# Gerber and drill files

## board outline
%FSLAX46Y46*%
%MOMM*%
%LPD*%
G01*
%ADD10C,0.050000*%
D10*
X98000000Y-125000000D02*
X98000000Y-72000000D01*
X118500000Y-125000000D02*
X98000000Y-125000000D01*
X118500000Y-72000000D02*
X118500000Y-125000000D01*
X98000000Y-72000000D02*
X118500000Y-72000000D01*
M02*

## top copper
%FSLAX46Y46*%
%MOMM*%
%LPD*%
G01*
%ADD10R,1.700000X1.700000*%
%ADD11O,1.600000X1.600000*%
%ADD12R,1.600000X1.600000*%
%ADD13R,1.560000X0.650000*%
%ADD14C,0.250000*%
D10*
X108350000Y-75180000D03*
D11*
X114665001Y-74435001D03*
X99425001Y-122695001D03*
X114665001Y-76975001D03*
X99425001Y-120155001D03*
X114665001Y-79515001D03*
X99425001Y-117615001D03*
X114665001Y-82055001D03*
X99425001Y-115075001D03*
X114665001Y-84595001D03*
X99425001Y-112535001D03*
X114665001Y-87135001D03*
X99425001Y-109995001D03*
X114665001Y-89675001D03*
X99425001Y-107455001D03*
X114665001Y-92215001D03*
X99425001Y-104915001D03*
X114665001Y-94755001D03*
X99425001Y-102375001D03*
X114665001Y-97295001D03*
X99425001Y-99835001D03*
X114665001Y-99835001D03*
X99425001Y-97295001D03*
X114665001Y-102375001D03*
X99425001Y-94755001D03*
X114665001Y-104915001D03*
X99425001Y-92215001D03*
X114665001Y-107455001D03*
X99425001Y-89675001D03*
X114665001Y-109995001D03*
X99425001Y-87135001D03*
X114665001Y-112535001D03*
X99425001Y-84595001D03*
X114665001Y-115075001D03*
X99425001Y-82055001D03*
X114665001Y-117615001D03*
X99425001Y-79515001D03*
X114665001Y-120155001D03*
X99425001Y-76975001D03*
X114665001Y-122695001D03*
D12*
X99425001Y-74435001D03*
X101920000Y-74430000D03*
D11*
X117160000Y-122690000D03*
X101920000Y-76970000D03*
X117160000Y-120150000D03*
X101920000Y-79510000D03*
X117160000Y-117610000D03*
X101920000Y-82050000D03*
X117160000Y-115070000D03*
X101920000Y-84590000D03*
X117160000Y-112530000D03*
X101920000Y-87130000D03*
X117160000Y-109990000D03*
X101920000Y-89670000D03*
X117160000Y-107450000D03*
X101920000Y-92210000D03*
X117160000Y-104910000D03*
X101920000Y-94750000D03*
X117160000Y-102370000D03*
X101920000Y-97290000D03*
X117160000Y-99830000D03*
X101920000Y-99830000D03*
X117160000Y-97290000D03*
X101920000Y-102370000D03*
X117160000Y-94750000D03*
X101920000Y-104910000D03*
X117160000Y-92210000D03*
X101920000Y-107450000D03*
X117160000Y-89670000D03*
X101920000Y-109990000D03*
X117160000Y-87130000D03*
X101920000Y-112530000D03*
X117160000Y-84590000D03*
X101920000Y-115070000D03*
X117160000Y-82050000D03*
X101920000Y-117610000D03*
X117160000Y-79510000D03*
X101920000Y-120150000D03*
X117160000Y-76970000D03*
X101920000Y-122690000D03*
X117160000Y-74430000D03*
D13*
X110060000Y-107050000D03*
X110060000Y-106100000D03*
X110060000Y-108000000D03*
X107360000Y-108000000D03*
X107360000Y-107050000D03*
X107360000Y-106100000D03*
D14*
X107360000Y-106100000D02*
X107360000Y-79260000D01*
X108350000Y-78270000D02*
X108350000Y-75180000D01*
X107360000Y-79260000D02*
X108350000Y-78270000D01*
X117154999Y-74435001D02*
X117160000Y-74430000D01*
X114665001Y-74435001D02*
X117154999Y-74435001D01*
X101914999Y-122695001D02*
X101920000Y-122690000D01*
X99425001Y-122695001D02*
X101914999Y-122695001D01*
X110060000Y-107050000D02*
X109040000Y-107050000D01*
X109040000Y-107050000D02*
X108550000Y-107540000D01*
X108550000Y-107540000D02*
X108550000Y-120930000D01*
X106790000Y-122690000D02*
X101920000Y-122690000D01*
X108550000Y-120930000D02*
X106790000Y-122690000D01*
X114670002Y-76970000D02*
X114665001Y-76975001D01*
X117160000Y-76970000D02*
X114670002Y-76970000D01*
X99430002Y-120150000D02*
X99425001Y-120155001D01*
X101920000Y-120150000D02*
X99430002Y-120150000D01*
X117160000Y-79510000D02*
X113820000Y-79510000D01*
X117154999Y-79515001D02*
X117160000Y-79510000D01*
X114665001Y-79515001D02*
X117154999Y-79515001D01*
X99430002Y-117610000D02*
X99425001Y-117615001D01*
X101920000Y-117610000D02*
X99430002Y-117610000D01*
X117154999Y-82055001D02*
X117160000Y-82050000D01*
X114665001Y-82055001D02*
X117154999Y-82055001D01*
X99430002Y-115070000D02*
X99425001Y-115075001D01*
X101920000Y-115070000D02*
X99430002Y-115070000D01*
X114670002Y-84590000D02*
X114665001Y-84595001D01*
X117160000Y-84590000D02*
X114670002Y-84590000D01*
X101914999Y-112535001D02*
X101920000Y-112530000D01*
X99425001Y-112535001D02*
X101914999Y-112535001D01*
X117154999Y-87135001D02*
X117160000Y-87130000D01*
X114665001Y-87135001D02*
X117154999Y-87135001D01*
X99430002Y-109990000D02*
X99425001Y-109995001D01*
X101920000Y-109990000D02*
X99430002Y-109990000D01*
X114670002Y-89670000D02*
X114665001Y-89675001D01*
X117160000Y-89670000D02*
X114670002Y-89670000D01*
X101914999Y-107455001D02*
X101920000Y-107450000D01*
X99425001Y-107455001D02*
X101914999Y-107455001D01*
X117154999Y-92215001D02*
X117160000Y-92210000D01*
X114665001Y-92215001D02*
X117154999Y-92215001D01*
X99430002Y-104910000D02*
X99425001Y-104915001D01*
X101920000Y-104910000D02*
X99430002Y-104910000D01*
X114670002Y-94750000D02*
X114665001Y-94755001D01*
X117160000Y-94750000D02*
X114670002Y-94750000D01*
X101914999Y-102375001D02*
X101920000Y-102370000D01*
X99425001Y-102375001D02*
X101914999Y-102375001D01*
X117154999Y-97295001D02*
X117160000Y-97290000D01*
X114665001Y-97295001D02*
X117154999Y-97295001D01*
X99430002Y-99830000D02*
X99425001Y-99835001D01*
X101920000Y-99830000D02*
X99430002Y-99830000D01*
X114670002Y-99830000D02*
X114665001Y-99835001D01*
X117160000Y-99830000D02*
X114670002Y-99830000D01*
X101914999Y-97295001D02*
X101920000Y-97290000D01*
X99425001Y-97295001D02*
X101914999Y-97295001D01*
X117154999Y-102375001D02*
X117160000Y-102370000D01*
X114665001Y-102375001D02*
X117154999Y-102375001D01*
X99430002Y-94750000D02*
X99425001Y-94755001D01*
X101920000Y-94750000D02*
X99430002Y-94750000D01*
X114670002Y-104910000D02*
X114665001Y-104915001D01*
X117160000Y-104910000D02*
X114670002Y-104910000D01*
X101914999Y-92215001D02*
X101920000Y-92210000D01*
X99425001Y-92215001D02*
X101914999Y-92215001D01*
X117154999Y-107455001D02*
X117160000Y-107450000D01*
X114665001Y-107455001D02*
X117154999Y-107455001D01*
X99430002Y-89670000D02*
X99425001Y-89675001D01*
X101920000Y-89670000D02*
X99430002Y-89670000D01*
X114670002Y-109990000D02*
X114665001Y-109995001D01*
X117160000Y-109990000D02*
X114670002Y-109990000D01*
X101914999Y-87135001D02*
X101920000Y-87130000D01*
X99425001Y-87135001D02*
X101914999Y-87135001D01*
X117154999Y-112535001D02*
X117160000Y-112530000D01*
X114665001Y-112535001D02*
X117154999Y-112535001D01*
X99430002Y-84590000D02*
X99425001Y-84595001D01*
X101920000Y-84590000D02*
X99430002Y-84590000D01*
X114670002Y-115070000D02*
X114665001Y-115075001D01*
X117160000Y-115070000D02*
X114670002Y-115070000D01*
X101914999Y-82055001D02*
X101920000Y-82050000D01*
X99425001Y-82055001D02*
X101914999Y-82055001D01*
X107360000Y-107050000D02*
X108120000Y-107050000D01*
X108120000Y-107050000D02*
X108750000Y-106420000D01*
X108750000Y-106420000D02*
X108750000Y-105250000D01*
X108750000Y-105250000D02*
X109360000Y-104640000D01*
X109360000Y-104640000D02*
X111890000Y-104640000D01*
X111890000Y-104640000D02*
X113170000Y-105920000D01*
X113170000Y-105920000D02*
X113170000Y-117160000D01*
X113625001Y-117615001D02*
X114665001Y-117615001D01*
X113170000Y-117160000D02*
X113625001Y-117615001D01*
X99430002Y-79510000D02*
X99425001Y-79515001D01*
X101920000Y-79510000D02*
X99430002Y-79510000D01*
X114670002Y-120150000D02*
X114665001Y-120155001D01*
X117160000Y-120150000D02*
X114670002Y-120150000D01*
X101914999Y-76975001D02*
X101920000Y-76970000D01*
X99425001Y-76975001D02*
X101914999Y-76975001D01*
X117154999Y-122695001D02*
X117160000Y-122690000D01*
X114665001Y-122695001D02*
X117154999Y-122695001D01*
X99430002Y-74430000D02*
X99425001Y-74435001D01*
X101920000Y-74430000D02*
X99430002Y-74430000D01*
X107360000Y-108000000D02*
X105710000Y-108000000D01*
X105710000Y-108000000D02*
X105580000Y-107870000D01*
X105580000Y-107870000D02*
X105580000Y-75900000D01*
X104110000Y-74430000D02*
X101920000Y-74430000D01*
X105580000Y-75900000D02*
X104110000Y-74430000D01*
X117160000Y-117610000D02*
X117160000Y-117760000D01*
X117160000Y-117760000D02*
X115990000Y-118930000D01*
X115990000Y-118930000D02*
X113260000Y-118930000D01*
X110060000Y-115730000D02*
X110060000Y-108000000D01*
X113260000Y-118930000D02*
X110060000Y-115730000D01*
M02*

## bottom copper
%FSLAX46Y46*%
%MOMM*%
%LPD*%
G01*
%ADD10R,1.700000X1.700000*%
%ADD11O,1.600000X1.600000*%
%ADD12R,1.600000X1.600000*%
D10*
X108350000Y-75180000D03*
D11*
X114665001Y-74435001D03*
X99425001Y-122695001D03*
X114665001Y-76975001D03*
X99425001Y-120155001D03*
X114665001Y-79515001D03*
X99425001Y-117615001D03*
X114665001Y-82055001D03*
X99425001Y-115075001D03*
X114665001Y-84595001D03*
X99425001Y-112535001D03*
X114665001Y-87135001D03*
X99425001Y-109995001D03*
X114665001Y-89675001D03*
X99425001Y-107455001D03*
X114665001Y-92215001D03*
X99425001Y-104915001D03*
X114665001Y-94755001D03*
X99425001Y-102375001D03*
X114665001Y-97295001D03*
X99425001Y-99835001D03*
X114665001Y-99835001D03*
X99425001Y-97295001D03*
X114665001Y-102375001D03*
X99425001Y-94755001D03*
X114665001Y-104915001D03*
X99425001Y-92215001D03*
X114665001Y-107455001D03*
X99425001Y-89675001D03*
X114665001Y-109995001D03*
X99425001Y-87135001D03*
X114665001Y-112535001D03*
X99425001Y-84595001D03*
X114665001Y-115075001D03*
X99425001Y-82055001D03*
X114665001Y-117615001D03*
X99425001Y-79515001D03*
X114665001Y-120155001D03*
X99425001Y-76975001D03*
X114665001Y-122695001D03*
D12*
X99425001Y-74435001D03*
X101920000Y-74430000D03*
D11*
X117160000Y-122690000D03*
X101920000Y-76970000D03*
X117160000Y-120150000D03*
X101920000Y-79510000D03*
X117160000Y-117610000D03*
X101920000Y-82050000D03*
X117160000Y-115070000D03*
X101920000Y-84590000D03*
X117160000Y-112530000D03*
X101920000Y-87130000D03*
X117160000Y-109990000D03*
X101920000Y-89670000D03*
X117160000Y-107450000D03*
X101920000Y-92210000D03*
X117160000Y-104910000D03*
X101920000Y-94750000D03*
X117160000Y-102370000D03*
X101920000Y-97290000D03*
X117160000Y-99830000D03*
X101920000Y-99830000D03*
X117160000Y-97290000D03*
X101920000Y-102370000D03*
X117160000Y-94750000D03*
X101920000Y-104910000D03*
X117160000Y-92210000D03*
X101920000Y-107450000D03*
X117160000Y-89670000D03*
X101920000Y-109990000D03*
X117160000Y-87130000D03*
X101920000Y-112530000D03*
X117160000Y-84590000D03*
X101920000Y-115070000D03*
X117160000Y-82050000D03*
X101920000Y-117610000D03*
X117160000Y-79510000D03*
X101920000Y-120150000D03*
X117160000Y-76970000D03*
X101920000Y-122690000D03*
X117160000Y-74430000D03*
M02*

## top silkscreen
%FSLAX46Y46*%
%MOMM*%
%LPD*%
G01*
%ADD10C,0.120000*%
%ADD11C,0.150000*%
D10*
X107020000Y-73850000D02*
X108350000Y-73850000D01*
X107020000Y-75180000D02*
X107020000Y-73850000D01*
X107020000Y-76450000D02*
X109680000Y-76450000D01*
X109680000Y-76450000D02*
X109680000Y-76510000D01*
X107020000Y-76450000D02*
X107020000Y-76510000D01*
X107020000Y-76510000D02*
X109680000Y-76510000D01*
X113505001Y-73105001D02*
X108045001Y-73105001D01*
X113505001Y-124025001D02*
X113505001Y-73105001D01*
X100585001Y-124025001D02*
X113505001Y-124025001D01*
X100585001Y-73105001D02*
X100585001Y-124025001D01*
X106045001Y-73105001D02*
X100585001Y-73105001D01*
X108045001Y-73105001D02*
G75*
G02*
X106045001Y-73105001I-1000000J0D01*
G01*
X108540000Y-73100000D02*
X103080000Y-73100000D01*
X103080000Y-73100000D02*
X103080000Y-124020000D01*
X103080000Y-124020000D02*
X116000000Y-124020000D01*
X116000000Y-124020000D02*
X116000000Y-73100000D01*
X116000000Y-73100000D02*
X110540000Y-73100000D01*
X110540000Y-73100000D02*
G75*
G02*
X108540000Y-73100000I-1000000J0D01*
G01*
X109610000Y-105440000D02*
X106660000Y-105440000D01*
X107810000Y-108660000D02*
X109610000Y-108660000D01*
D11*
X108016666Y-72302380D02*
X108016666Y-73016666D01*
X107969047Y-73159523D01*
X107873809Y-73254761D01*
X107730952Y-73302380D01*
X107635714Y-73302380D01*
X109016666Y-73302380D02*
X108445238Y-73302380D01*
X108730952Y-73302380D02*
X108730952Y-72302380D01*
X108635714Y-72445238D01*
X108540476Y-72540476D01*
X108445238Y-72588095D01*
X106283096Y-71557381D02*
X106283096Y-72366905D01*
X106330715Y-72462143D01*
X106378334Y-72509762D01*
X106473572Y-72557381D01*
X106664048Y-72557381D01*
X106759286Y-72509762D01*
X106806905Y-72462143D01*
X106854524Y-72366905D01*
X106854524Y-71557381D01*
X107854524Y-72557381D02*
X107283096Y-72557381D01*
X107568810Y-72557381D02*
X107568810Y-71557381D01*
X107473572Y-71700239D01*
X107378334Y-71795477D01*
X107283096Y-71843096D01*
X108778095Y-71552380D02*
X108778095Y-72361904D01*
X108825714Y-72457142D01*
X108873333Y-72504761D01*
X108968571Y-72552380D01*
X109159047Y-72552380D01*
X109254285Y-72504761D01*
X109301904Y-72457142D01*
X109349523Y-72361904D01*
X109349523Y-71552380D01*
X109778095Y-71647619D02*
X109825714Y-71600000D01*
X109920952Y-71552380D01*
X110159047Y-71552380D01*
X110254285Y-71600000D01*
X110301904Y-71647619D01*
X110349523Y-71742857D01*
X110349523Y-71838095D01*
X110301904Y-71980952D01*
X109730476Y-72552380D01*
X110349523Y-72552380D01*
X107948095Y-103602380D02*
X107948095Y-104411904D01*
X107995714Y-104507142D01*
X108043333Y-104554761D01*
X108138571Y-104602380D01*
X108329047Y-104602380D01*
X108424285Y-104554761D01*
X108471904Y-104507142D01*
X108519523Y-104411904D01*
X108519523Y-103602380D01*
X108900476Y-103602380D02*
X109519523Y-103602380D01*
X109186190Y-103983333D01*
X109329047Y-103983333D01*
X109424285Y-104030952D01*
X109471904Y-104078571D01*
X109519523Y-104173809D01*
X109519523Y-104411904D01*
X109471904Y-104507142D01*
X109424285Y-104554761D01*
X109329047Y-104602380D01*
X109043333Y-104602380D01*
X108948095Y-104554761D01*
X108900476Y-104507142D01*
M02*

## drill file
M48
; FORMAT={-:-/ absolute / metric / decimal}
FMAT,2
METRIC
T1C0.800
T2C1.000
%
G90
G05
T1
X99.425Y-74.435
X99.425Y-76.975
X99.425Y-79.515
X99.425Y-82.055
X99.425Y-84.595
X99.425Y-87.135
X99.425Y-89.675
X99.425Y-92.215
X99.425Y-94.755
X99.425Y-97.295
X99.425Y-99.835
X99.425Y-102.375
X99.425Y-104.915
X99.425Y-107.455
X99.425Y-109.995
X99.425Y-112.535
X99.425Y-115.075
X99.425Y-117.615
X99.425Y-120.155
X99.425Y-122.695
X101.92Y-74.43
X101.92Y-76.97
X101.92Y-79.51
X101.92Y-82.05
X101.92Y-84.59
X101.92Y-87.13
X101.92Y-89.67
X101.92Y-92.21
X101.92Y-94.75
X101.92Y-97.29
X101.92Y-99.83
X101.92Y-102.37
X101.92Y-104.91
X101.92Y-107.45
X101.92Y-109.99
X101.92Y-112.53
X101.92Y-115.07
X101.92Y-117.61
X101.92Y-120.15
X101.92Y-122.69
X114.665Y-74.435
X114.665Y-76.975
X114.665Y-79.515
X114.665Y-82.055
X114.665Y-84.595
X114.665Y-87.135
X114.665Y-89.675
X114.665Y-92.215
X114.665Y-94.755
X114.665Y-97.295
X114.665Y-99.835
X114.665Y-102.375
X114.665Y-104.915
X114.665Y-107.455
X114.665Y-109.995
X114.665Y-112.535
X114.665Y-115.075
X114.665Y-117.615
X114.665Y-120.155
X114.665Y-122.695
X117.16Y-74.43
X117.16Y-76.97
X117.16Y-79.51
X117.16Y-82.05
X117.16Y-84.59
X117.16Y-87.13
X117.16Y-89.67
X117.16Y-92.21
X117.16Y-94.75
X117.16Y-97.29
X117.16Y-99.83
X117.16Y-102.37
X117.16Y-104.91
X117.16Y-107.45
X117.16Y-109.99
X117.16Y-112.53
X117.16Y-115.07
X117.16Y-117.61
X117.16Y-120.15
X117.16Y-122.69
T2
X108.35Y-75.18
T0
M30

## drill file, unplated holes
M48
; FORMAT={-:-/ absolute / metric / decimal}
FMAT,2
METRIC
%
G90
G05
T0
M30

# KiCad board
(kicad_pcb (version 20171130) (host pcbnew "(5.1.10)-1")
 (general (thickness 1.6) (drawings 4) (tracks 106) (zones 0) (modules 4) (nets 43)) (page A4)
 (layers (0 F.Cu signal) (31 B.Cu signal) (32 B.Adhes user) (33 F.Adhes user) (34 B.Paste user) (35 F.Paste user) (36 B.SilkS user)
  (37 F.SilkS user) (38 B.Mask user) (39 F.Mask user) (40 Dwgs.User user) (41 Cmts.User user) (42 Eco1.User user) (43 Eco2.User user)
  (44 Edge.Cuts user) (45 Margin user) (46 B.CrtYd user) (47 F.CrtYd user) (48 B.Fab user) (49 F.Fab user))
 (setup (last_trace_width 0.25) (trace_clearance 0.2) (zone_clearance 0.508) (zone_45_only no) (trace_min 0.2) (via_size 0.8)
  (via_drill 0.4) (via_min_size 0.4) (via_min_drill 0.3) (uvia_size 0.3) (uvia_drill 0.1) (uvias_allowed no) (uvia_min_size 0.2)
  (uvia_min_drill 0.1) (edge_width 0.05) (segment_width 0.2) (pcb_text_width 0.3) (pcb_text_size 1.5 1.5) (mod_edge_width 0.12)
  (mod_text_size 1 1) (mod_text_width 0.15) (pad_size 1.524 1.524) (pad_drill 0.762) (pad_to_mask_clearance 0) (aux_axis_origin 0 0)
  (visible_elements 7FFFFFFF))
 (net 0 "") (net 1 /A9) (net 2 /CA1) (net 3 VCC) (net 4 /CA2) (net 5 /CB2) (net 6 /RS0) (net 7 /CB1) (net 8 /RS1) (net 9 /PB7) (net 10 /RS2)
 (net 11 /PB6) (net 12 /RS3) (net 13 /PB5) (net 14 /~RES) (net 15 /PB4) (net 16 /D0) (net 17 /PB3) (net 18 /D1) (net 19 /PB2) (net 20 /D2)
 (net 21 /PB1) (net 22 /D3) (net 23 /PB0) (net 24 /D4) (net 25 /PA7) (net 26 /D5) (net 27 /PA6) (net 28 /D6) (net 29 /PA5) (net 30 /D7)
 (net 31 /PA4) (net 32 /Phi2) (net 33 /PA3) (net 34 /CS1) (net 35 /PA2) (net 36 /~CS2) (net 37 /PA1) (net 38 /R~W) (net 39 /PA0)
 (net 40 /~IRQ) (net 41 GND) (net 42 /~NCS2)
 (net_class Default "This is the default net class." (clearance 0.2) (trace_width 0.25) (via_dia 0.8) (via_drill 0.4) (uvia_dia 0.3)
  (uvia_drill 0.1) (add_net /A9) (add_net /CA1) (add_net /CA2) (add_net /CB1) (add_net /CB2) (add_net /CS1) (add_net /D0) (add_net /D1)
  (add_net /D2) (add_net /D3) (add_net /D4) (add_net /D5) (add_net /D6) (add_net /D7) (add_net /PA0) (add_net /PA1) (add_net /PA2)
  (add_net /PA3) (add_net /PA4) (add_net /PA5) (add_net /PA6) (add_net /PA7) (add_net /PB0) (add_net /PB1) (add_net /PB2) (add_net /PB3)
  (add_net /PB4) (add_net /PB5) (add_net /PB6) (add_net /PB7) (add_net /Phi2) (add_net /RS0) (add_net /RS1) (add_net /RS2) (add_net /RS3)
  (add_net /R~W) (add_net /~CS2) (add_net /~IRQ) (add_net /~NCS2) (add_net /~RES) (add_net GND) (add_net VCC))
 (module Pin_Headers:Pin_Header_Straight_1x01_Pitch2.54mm (layer F.Cu) (at 108.35 75.18)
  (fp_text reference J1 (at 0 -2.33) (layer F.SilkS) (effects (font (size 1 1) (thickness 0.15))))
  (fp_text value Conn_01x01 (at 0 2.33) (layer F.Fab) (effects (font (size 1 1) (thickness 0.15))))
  (fp_line (start -1.33 -1.33) (end 0 -1.33) (layer F.SilkS) (width 0.12))
  (fp_line (start -1.33 0) (end -1.33 -1.33) (layer F.SilkS) (width 0.12))
  (fp_line (start -1.33 1.27) (end 1.33 1.27) (layer F.SilkS) (width 0.12))
  (fp_line (start 1.33 1.27) (end 1.33 1.33) (layer F.SilkS) (width 0.12))
  (fp_line (start -1.33 1.27) (end -1.33 1.33) (layer F.SilkS) (width 0.12))
  (fp_line (start -1.33 1.33) (end 1.33 1.33) (layer F.SilkS) (width 0.12))
  (pad 1 thru_hole rect (at 0 0) (size 1.7 1.7) (drill 1) (layers *.Cu *.Mask) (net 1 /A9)))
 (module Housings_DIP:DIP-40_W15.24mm (layer F.Cu) (at 99.425001 74.435001)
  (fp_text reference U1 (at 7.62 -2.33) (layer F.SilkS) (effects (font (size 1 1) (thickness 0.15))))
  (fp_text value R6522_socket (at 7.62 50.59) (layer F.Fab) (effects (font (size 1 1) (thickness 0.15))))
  (fp_line (start 14.08 -1.33) (end 8.62 -1.33) (layer F.SilkS) (width 0.12))
  (fp_line (start 14.08 49.59) (end 14.08 -1.33) (layer F.SilkS) (width 0.12))
  (fp_line (start 1.16 49.59) (end 14.08 49.59) (layer F.SilkS) (width 0.12))
  (fp_line (start 1.16 -1.33) (end 1.16 49.59) (layer F.SilkS) (width 0.12))
  (fp_line (start 6.62 -1.33) (end 1.16 -1.33) (layer F.SilkS) (width 0.12))
  (fp_arc (start 7.62 -1.33) (end 6.62 -1.33) (angle -180) (layer F.SilkS) (width 0.12))
  (pad 40 thru_hole oval (at 15.24 0) (size 1.6 1.6) (drill 0.8) (layers *.Cu *.Mask) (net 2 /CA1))
  (pad 20 thru_hole oval (at 0 48.26) (size 1.6 1.6) (drill 0.8) (layers *.Cu *.Mask) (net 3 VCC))
  (pad 39 thru_hole oval (at 15.24 2.54) (size 1.6 1.6) (drill 0.8) (layers *.Cu *.Mask) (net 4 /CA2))
  (pad 19 thru_hole oval (at 0 45.72) (size 1.6 1.6) (drill 0.8) (layers *.Cu *.Mask) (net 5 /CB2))
  (pad 38 thru_hole oval (at 15.24 5.08) (size 1.6 1.6) (drill 0.8) (layers *.Cu *.Mask) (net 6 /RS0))
  (pad 18 thru_hole oval (at 0 43.18) (size 1.6 1.6) (drill 0.8) (layers *.Cu *.Mask) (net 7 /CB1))
  (pad 37 thru_hole oval (at 15.24 7.62) (size 1.6 1.6) (drill 0.8) (layers *.Cu *.Mask) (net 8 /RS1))
  (pad 17 thru_hole oval (at 0 40.64) (size 1.6 1.6) (drill 0.8) (layers *.Cu *.Mask) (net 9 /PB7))
  (pad 36 thru_hole oval (at 15.24 10.16) (size 1.6 1.6) (drill 0.8) (layers *.Cu *.Mask) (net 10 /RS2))
  (pad 16 thru_hole oval (at 0 38.1) (size 1.6 1.6) (drill 0.8) (layers *.Cu *.Mask) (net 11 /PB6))
  (pad 35 thru_hole oval (at 15.24 12.7) (size 1.6 1.6) (drill 0.8) (layers *.Cu *.Mask) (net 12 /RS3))
  (pad 15 thru_hole oval (at 0 35.56) (size 1.6 1.6) (drill 0.8) (layers *.Cu *.Mask) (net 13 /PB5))
  (pad 34 thru_hole oval (at 15.24 15.24) (size 1.6 1.6) (drill 0.8) (layers *.Cu *.Mask) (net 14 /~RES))
  (pad 14 thru_hole oval (at 0 33.02) (size 1.6 1.6) (drill 0.8) (layers *.Cu *.Mask) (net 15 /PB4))
  (pad 33 thru_hole oval (at 15.24 17.78) (size 1.6 1.6) (drill 0.8) (layers *.Cu *.Mask) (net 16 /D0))
  (pad 13 thru_hole oval (at 0 30.48) (size 1.6 1.6) (drill 0.8) (layers *.Cu *.Mask) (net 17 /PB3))
  (pad 32 thru_hole oval (at 15.24 20.32) (size 1.6 1.6) (drill 0.8) (layers *.Cu *.Mask) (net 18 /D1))
  (pad 12 thru_hole oval (at 0 27.94) (size 1.6 1.6) (drill 0.8) (layers *.Cu *.Mask) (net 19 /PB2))
  (pad 31 thru_hole oval (at 15.24 22.86) (size 1.6 1.6) (drill 0.8) (layers *.Cu *.Mask) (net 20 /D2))
  (pad 11 thru_hole oval (at 0 25.4) (size 1.6 1.6) (drill 0.8) (layers *.Cu *.Mask) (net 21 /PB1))
  (pad 30 thru_hole oval (at 15.24 25.4) (size 1.6 1.6) (drill 0.8) (layers *.Cu *.Mask) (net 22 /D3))
  (pad 10 thru_hole oval (at 0 22.86) (size 1.6 1.6) (drill 0.8) (layers *.Cu *.Mask) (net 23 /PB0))
  (pad 29 thru_hole oval (at 15.24 27.94) (size 1.6 1.6) (drill 0.8) (layers *.Cu *.Mask) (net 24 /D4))
  (pad 9 thru_hole oval (at 0 20.32) (size 1.6 1.6) (drill 0.8) (layers *.Cu *.Mask) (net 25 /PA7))
  (pad 28 thru_hole oval (at 15.24 30.48) (size 1.6 1.6) (drill 0.8) (layers *.Cu *.Mask) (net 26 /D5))
  (pad 8 thru_hole oval (at 0 17.78) (size 1.6 1.6) (drill 0.8) (layers *.Cu *.Mask) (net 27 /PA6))
  (pad 27 thru_hole oval (at 15.24 33.02) (size 1.6 1.6) (drill 0.8) (layers *.Cu *.Mask) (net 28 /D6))
  (pad 7 thru_hole oval (at 0 15.24) (size 1.6 1.6) (drill 0.8) (layers *.Cu *.Mask) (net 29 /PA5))
  (pad 26 thru_hole oval (at 15.24 35.56) (size 1.6 1.6) (drill 0.8) (layers *.Cu *.Mask) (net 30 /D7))
  (pad 6 thru_hole oval (at 0 12.7) (size 1.6 1.6) (drill 0.8) (layers *.Cu *.Mask) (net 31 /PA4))
  (pad 25 thru_hole oval (at 15.24 38.1) (size 1.6 1.6) (drill 0.8) (layers *.Cu *.Mask) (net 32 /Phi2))
  (pad 5 thru_hole oval (at 0 10.16) (size 1.6 1.6) (drill 0.8) (layers *.Cu *.Mask) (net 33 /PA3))
  (pad 24 thru_hole oval (at 15.24 40.64) (size 1.6 1.6) (drill 0.8) (layers *.Cu *.Mask) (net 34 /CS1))
  (pad 4 thru_hole oval (at 0 7.62) (size 1.6 1.6) (drill 0.8) (layers *.Cu *.Mask) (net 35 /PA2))
  (pad 23 thru_hole oval (at 15.24 43.18) (size 1.6 1.6) (drill 0.8) (layers *.Cu *.Mask) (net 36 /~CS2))
  (pad 3 thru_hole oval (at 0 5.08) (size 1.6 1.6) (drill 0.8) (layers *.Cu *.Mask) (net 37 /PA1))
  (pad 22 thru_hole oval (at 15.24 45.72) (size 1.6 1.6) (drill 0.8) (layers *.Cu *.Mask) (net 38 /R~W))
  (pad 2 thru_hole oval (at 0 2.54) (size 1.6 1.6) (drill 0.8) (layers *.Cu *.Mask) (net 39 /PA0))
  (pad 21 thru_hole oval (at 15.24 48.26) (size 1.6 1.6) (drill 0.8) (layers *.Cu *.Mask) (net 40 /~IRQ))
  (pad 1 thru_hole rect (at 0 0) (size 1.6 1.6) (drill 0.8) (layers *.Cu *.Mask) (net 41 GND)))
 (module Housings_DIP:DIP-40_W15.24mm (layer F.Cu) (at 101.92 74.43)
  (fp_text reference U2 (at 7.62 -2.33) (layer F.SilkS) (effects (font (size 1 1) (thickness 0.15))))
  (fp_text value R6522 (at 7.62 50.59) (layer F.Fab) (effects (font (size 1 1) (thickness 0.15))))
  (fp_line (start 6.62 -1.33) (end 1.16 -1.33) (layer F.SilkS) (width 0.12))
  (fp_line (start 1.16 -1.33) (end 1.16 49.59) (layer F.SilkS) (width 0.12))
  (fp_line (start 1.16 49.59) (end 14.08 49.59) (layer F.SilkS) (width 0.12))
  (fp_line (start 14.08 49.59) (end 14.08 -1.33) (layer F.SilkS) (width 0.12))
  (fp_line (start 14.08 -1.33) (end 8.62 -1.33) (layer F.SilkS) (width 0.12))
  (fp_arc (start 7.62 -1.33) (end 6.62 -1.33) (angle -180) (layer F.SilkS) (width 0.12))
  (pad 1 thru_hole rect (at 0 0) (size 1.6 1.6) (drill 0.8) (layers *.Cu *.Mask) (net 41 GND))
  (pad 21 thru_hole oval (at 15.24 48.26) (size 1.6 1.6) (drill 0.8) (layers *.Cu *.Mask) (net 40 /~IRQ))
  (pad 2 thru_hole oval (at 0 2.54) (size 1.6 1.6) (drill 0.8) (layers *.Cu *.Mask) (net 39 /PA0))
  (pad 22 thru_hole oval (at 15.24 45.72) (size 1.6 1.6) (drill 0.8) (layers *.Cu *.Mask) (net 38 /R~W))
  (pad 3 thru_hole oval (at 0 5.08) (size 1.6 1.6) (drill 0.8) (layers *.Cu *.Mask) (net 37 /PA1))
  (pad 23 thru_hole oval (at 15.24 43.18) (size 1.6 1.6) (drill 0.8) (layers *.Cu *.Mask) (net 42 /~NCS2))
  (pad 4 thru_hole oval (at 0 7.62) (size 1.6 1.6) (drill 0.8) (layers *.Cu *.Mask) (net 35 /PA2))
  (pad 24 thru_hole oval (at 15.24 40.64) (size 1.6 1.6) (drill 0.8) (layers *.Cu *.Mask) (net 34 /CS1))
  (pad 5 thru_hole oval (at 0 10.16) (size 1.6 1.6) (drill 0.8) (layers *.Cu *.Mask) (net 33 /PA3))
  (pad 25 thru_hole oval (at 15.24 38.1) (size 1.6 1.6) (drill 0.8) (layers *.Cu *.Mask) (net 32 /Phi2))
  (pad 6 thru_hole oval (at 0 12.7) (size 1.6 1.6) (drill 0.8) (layers *.Cu *.Mask) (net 31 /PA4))
  (pad 26 thru_hole oval (at 15.24 35.56) (size 1.6 1.6) (drill 0.8) (layers *.Cu *.Mask) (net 30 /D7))
  (pad 7 thru_hole oval (at 0 15.24) (size 1.6 1.6) (drill 0.8) (layers *.Cu *.Mask) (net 29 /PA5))
  (pad 27 thru_hole oval (at 15.24 33.02) (size 1.6 1.6) (drill 0.8) (layers *.Cu *.Mask) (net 28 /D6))
  (pad 8 thru_hole oval (at 0 17.78) (size 1.6 1.6) (drill 0.8) (layers *.Cu *.Mask) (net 27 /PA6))
  (pad 28 thru_hole oval (at 15.24 30.48) (size 1.6 1.6) (drill 0.8) (layers *.Cu *.Mask) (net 26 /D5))
  (pad 9 thru_hole oval (at 0 20.32) (size 1.6 1.6) (drill 0.8) (layers *.Cu *.Mask) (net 25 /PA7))
  (pad 29 thru_hole oval (at 15.24 27.94) (size 1.6 1.6) (drill 0.8) (layers *.Cu *.Mask) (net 24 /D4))
  (pad 10 thru_hole oval (at 0 22.86) (size 1.6 1.6) (drill 0.8) (layers *.Cu *.Mask) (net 23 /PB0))
  (pad 30 thru_hole oval (at 15.24 25.4) (size 1.6 1.6) (drill 0.8) (layers *.Cu *.Mask) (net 22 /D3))
  (pad 11 thru_hole oval (at 0 25.4) (size 1.6 1.6) (drill 0.8) (layers *.Cu *.Mask) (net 21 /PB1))
  (pad 31 thru_hole oval (at 15.24 22.86) (size 1.6 1.6) (drill 0.8) (layers *.Cu *.Mask) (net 20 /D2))
  (pad 12 thru_hole oval (at 0 27.94) (size 1.6 1.6) (drill 0.8) (layers *.Cu *.Mask) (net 19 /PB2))
  (pad 32 thru_hole oval (at 15.24 20.32) (size 1.6 1.6) (drill 0.8) (layers *.Cu *.Mask) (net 18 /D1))
  (pad 13 thru_hole oval (at 0 30.48) (size 1.6 1.6) (drill 0.8) (layers *.Cu *.Mask) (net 17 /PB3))
  (pad 33 thru_hole oval (at 15.24 17.78) (size 1.6 1.6) (drill 0.8) (layers *.Cu *.Mask) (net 16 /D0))
  (pad 14 thru_hole oval (at 0 33.02) (size 1.6 1.6) (drill 0.8) (layers *.Cu *.Mask) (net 15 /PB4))
  (pad 34 thru_hole oval (at 15.24 15.24) (size 1.6 1.6) (drill 0.8) (layers *.Cu *.Mask) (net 14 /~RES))
  (pad 15 thru_hole oval (at 0 35.56) (size 1.6 1.6) (drill 0.8) (layers *.Cu *.Mask) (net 13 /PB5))
  (pad 35 thru_hole oval (at 15.24 12.7) (size 1.6 1.6) (drill 0.8) (layers *.Cu *.Mask) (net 12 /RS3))
  (pad 16 thru_hole oval (at 0 38.1) (size 1.6 1.6) (drill 0.8) (layers *.Cu *.Mask) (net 11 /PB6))
  (pad 36 thru_hole oval (at 15.24 10.16) (size 1.6 1.6) (drill 0.8) (layers *.Cu *.Mask) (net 10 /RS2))
  (pad 17 thru_hole oval (at 0 40.64) (size 1.6 1.6) (drill 0.8) (layers *.Cu *.Mask) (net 9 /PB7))
  (pad 37 thru_hole oval (at 15.24 7.62) (size 1.6 1.6) (drill 0.8) (layers *.Cu *.Mask) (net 8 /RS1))
  (pad 18 thru_hole oval (at 0 43.18) (size 1.6 1.6) (drill 0.8) (layers *.Cu *.Mask) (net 7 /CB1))
  (pad 38 thru_hole oval (at 15.24 5.08) (size 1.6 1.6) (drill 0.8) (layers *.Cu *.Mask) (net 6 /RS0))
  (pad 19 thru_hole oval (at 0 45.72) (size 1.6 1.6) (drill 0.8) (layers *.Cu *.Mask) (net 5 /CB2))
  (pad 39 thru_hole oval (at 15.24 2.54) (size 1.6 1.6) (drill 0.8) (layers *.Cu *.Mask) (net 4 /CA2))
  (pad 20 thru_hole oval (at 0 48.26) (size 1.6 1.6) (drill 0.8) (layers *.Cu *.Mask) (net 3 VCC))
  (pad 40 thru_hole oval (at 15.24 0) (size 1.6 1.6) (drill 0.8) (layers *.Cu *.Mask) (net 2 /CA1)))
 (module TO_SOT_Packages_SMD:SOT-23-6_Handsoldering (layer F.Cu) (at 108.71 107.05)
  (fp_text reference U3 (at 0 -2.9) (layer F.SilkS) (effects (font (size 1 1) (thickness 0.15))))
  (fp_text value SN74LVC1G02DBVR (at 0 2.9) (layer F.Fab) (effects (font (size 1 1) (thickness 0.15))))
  (fp_line (start 0.9 -1.61) (end -2.05 -1.61) (layer F.SilkS) (width 0.12))
  (fp_line (start -0.9 1.61) (end 0.9 1.61) (layer F.SilkS) (width 0.12))
  (pad 5 smd rect (at 1.35 0) (size 1.56 0.65) (layers F.Cu F.Paste F.Mask) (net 3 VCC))
  (pad 6 smd rect (at 1.35 -0.95) (size 1.56 0.65) (layers F.Cu F.Paste F.Mask))
  (pad 4 smd rect (at 1.35 0.95) (size 1.56 0.65) (layers F.Cu F.Paste F.Mask) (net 42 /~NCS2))
  (pad 3 smd rect (at -1.35 0.95) (size 1.56 0.65) (layers F.Cu F.Paste F.Mask) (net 41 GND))
  (pad 2 smd rect (at -1.35 0) (size 1.56 0.65) (layers F.Cu F.Paste F.Mask) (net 36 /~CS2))
  (pad 1 smd rect (at -1.35 -0.95) (size 1.56 0.65) (layers F.Cu F.Paste F.Mask) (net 1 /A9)))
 (gr_line (start 98 125) (end 98 72) (layer Edge.Cuts) (width 0.05))
 (gr_line (start 118.5 125) (end 98 125) (layer Edge.Cuts) (width 0.05))
 (gr_line (start 118.5 72) (end 118.5 125) (layer Edge.Cuts) (width 0.05))
 (gr_line (start 98 72) (end 118.5 72) (layer Edge.Cuts) (width 0.05))
 (segment (start 107.36 106.1) (end 107.36 79.26) (width 0.25) (layer F.Cu) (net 1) (status 10))
 (segment (start 108.35 78.27) (end 108.35 75.18) (width 0.25) (layer F.Cu) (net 1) (status 20))
 (segment (start 107.36 79.26) (end 108.35 78.27) (width 0.25) (layer F.Cu) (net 1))
 (segment (start 117.154999 74.435001) (end 117.16 74.43) (width 0.25) (layer F.Cu) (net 2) (status 30))
 (segment (start 114.665001 74.435001) (end 117.154999 74.435001) (width 0.25) (layer F.Cu) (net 2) (status 30))
 (segment (start 101.914999 122.695001) (end 101.92 122.69) (width 0.25) (layer F.Cu) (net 3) (status 30))
 (segment (start 99.425001 122.695001) (end 101.914999 122.695001) (width 0.25) (layer F.Cu) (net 3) (status 30))
 (segment (start 110.06 107.05) (end 109.04 107.05) (width 0.25) (layer F.Cu) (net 3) (status 10))
 (segment (start 109.04 107.05) (end 108.55 107.54) (width 0.25) (layer F.Cu) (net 3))
 (segment (start 108.55 107.54) (end 108.55 120.93) (width 0.25) (layer F.Cu) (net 3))
 (segment (start 106.79 122.69) (end 101.92 122.69) (width 0.25) (layer F.Cu) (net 3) (status 20))
 (segment (start 108.55 120.93) (end 106.79 122.69) (width 0.25) (layer F.Cu) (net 3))
 (segment (start 114.670002 76.97) (end 114.665001 76.975001) (width 0.25) (layer F.Cu) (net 4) (status 30))
 (segment (start 117.16 76.97) (end 114.670002 76.97) (width 0.25) (layer F.Cu) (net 4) (status 30))
 (segment (start 99.430002 120.15) (end 99.425001 120.155001) (width 0.25) (layer F.Cu) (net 5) (status 30))
 (segment (start 101.92 120.15) (end 99.430002 120.15) (width 0.25) (layer F.Cu) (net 5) (status 30))
 (segment (start 117.16 79.51) (end 113.82 79.51) (width 0.25) (layer F.Cu) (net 6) (status 10))
 (segment (start 117.154999 79.515001) (end 117.16 79.51) (width 0.25) (layer F.Cu) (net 6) (status 30))
 (segment (start 114.665001 79.515001) (end 117.154999 79.515001) (width 0.25) (layer F.Cu) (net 6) (status 30))
 (segment (start 99.430002 117.61) (end 99.425001 117.615001) (width 0.25) (layer F.Cu) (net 7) (status 30))
 (segment (start 101.92 117.61) (end 99.430002 117.61) (width 0.25) (layer F.Cu) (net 7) (status 30))
 (segment (start 117.154999 82.055001) (end 117.16 82.05) (width 0.25) (layer F.Cu) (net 8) (status 30))
 (segment (start 114.665001 82.055001) (end 117.154999 82.055001) (width 0.25) (layer F.Cu) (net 8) (status 30))
 (segment (start 99.430002 115.07) (end 99.425001 115.075001) (width 0.25) (layer F.Cu) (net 9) (status 30))
 (segment (start 101.92 115.07) (end 99.430002 115.07) (width 0.25) (layer F.Cu) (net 9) (status 30))
 (segment (start 114.670002 84.59) (end 114.665001 84.595001) (width 0.25) (layer F.Cu) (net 10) (status 30))
 (segment (start 117.16 84.59) (end 114.670002 84.59) (width 0.25) (layer F.Cu) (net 10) (status 30))
 (segment (start 101.914999 112.535001) (end 101.92 112.53) (width 0.25) (layer F.Cu) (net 11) (status 30))
 (segment (start 99.425001 112.535001) (end 101.914999 112.535001) (width 0.25) (layer F.Cu) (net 11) (status 30))
 (segment (start 117.154999 87.135001) (end 117.16 87.13) (width 0.25) (layer F.Cu) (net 12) (status 30))
 (segment (start 114.665001 87.135001) (end 117.154999 87.135001) (width 0.25) (layer F.Cu) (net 12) (status 30))
 (segment (start 99.430002 109.99) (end 99.425001 109.995001) (width 0.25) (layer F.Cu) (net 13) (status 30))
 (segment (start 101.92 109.99) (end 99.430002 109.99) (width 0.25) (layer F.Cu) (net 13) (status 30))
 (segment (start 114.670002 89.67) (end 114.665001 89.675001) (width 0.25) (layer F.Cu) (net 14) (status 30))
 (segment (start 117.16 89.67) (end 114.670002 89.67) (width 0.25) (layer F.Cu) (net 14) (status 30))
 (segment (start 101.914999 107.455001) (end 101.92 107.45) (width 0.25) (layer F.Cu) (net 15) (status 30))
 (segment (start 99.425001 107.455001) (end 101.914999 107.455001) (width 0.25) (layer F.Cu) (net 15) (status 30))
 (segment (start 117.154999 92.215001) (end 117.16 92.21) (width 0.25) (layer F.Cu) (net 16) (status 30))
 (segment (start 114.665001 92.215001) (end 117.154999 92.215001) (width 0.25) (layer F.Cu) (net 16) (status 30))
 (segment (start 99.430002 104.91) (end 99.425001 104.915001) (width 0.25) (layer F.Cu) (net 17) (status 30))
 (segment (start 101.92 104.91) (end 99.430002 104.91) (width 0.25) (layer F.Cu) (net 17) (status 30))
 (segment (start 114.670002 94.75) (end 114.665001 94.755001) (width 0.25) (layer F.Cu) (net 18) (status 30))
 (segment (start 117.16 94.75) (end 114.670002 94.75) (width 0.25) (layer F.Cu) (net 18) (status 30))
 (segment (start 101.914999 102.375001) (end 101.92 102.37) (width 0.25) (layer F.Cu) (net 19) (status 30))
 (segment (start 99.425001 102.375001) (end 101.914999 102.375001) (width 0.25) (layer F.Cu) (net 19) (status 30))
 (segment (start 117.154999 97.295001) (end 117.16 97.29) (width 0.25) (layer F.Cu) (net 20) (status 30))
 (segment (start 114.665001 97.295001) (end 117.154999 97.295001) (width 0.25) (layer F.Cu) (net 20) (status 30))
 (segment (start 99.430002 99.83) (end 99.425001 99.835001) (width 0.25) (layer F.Cu) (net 21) (status 30))
 (segment (start 101.92 99.83) (end 99.430002 99.83) (width 0.25) (layer F.Cu) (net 21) (status 30))
 (segment (start 114.670002 99.83) (end 114.665001 99.835001) (width 0.25) (layer F.Cu) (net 22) (status 30))
 (segment (start 117.16 99.83) (end 114.670002 99.83) (width 0.25) (layer F.Cu) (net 22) (status 30))
 (segment (start 101.914999 97.295001) (end 101.92 97.29) (width 0.25) (layer F.Cu) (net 23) (status 30))
 (segment (start 99.425001 97.295001) (end 101.914999 97.295001) (width 0.25) (layer F.Cu) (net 23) (status 30))
 (segment (start 117.154999 102.375001) (end 117.16 102.37) (width 0.25) (layer F.Cu) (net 24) (status 30))
 (segment (start 114.665001 102.375001) (end 117.154999 102.375001) (width 0.25) (layer F.Cu) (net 24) (status 30))
 (segment (start 99.430002 94.75) (end 99.425001 94.755001) (width 0.25) (layer F.Cu) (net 25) (status 30))
 (segment (start 101.92 94.75) (end 99.430002 94.75) (width 0.25) (layer F.Cu) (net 25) (status 30))
 (segment (start 114.670002 104.91) (end 114.665001 104.915001) (width 0.25) (layer F.Cu) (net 26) (status 30))
 (segment (start 117.16 104.91) (end 114.670002 104.91) (width 0.25) (layer F.Cu) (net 26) (status 30))
 (segment (start 101.914999 92.215001) (end 101.92 92.21) (width 0.25) (layer F.Cu) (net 27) (status 30))
 (segment (start 99.425001 92.215001) (end 101.914999 92.215001) (width 0.25) (layer F.Cu) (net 27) (status 30))
 (segment (start 117.154999 107.455001) (end 117.16 107.45) (width 0.25) (layer F.Cu) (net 28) (status 30))
 (segment (start 114.665001 107.455001) (end 117.154999 107.455001) (width 0.25) (layer F.Cu) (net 28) (status 30))
 (segment (start 99.430002 89.67) (end 99.425001 89.675001) (width 0.25) (layer F.Cu) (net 29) (status 30))
 (segment (start 101.92 89.67) (end 99.430002 89.67) (width 0.25) (layer F.Cu) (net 29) (status 30))
 (segment (start 114.670002 109.99) (end 114.665001 109.995001) (width 0.25) (layer F.Cu) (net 30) (status 30))
 (segment (start 117.16 109.99) (end 114.670002 109.99) (width 0.25) (layer F.Cu) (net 30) (status 30))
 (segment (start 101.914999 87.135001) (end 101.92 87.13) (width 0.25) (layer F.Cu) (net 31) (status 30))
 (segment (start 99.425001 87.135001) (end 101.914999 87.135001) (width 0.25) (layer F.Cu) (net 31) (status 30))
 (segment (start 117.154999 112.535001) (end 117.16 112.53) (width 0.25) (layer F.Cu) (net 32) (status 30))
 (segment (start 114.665001 112.535001) (end 117.154999 112.535001) (width 0.25) (layer F.Cu) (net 32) (status 30))
 (segment (start 99.430002 84.59) (end 99.425001 84.595001) (width 0.25) (layer F.Cu) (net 33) (status 30))
 (segment (start 101.92 84.59) (end 99.430002 84.59) (width 0.25) (layer F.Cu) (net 33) (status 30))
 (segment (start 114.670002 115.07) (end 114.665001 115.075001) (width 0.25) (layer F.Cu) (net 34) (status 30))
 (segment (start 117.16 115.07) (end 114.670002 115.07) (width 0.25) (layer F.Cu) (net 34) (status 30))
 (segment (start 101.914999 82.055001) (end 101.92 82.05) (width 0.25) (layer F.Cu) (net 35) (status 30))
 (segment (start 99.425001 82.055001) (end 101.914999 82.055001) (width 0.25) (layer F.Cu) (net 35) (status 30))
 (segment (start 107.36 107.05) (end 108.12 107.05) (width 0.25) (layer F.Cu) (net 36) (status 30))
 (segment (start 108.12 107.05) (end 108.75 106.42) (width 0.25) (layer F.Cu) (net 36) (status 10))
 (segment (start 108.75 106.42) (end 108.75 105.25) (width 0.25) (layer F.Cu) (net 36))
 (segment (start 108.75 105.25) (end 109.36 104.64) (width 0.25) (layer F.Cu) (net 36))
 (segment (start 109.36 104.64) (end 111.89 104.64) (width 0.25) (layer F.Cu) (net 36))
 (segment (start 111.89 104.64) (end 113.17 105.92) (width 0.25) (layer F.Cu) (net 36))
 (segment (start 113.17 105.92) (end 113.17 117.16) (width 0.25) (layer F.Cu) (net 36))
 (segment (start 113.625001 117.615001) (end 114.665001 117.615001) (width 0.25) (layer F.Cu) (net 36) (status 20))
 (segment (start 113.17 117.16) (end 113.625001 117.615001) (width 0.25) (layer F.Cu) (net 36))
 (segment (start 99.430002 79.51) (end 99.425001 79.515001) (width 0.25) (layer F.Cu) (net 37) (status 30))
 (segment (start 101.92 79.51) (end 99.430002 79.51) (width 0.25) (layer F.Cu) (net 37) (status 30))
 (segment (start 114.670002 120.15) (end 114.665001 120.155001) (width 0.25) (layer F.Cu) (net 38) (status 30))
 (segment (start 117.16 120.15) (end 114.670002 120.15) (width 0.25) (layer F.Cu) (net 38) (status 30))
 (segment (start 101.914999 76.975001) (end 101.92 76.97) (width 0.25) (layer F.Cu) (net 39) (status 30))
 (segment (start 99.425001 76.975001) (end 101.914999 76.975001) (width 0.25) (layer F.Cu) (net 39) (status 30))
 (segment (start 117.154999 122.695001) (end 117.16 122.69) (width 0.25) (layer F.Cu) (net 40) (status 30))
 (segment (start 114.665001 122.695001) (end 117.154999 122.695001) (width 0.25) (layer F.Cu) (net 40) (status 30))
 (segment (start 99.430002 74.43) (end 99.425001 74.435001) (width 0.25) (layer F.Cu) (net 41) (status 30))
 (segment (start 101.92 74.43) (end 99.430002 74.43) (width 0.25) (layer F.Cu) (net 41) (status 30))
 (segment (start 107.36 108) (end 105.71 108) (width 0.25) (layer F.Cu) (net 41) (status 10))
 (segment (start 105.71 108) (end 105.58 107.87) (width 0.25) (layer F.Cu) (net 41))
 (segment (start 105.58 107.87) (end 105.58 75.9) (width 0.25) (layer F.Cu) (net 41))
 (segment (start 104.11 74.43) (end 101.92 74.43) (width 0.25) (layer F.Cu) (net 41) (status 20))
 (segment (start 105.58 75.9) (end 104.11 74.43) (width 0.25) (layer F.Cu) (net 41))
 (segment (start 117.16 117.61) (end 117.16 117.76) (width 0.25) (layer F.Cu) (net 42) (status 30))
 (segment (start 117.16 117.76) (end 115.99 118.93) (width 0.25) (layer F.Cu) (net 42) (status 10))
 (segment (start 115.99 118.93) (end 113.26 118.93) (width 0.25) (layer F.Cu) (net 42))
 (segment (start 110.06 115.73) (end 110.06 108) (width 0.25) (layer F.Cu) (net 42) (status 20))
 (segment (start 113.26 118.93) (end 110.06 115.73) (width 0.25) (layer F.Cu) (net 42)))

